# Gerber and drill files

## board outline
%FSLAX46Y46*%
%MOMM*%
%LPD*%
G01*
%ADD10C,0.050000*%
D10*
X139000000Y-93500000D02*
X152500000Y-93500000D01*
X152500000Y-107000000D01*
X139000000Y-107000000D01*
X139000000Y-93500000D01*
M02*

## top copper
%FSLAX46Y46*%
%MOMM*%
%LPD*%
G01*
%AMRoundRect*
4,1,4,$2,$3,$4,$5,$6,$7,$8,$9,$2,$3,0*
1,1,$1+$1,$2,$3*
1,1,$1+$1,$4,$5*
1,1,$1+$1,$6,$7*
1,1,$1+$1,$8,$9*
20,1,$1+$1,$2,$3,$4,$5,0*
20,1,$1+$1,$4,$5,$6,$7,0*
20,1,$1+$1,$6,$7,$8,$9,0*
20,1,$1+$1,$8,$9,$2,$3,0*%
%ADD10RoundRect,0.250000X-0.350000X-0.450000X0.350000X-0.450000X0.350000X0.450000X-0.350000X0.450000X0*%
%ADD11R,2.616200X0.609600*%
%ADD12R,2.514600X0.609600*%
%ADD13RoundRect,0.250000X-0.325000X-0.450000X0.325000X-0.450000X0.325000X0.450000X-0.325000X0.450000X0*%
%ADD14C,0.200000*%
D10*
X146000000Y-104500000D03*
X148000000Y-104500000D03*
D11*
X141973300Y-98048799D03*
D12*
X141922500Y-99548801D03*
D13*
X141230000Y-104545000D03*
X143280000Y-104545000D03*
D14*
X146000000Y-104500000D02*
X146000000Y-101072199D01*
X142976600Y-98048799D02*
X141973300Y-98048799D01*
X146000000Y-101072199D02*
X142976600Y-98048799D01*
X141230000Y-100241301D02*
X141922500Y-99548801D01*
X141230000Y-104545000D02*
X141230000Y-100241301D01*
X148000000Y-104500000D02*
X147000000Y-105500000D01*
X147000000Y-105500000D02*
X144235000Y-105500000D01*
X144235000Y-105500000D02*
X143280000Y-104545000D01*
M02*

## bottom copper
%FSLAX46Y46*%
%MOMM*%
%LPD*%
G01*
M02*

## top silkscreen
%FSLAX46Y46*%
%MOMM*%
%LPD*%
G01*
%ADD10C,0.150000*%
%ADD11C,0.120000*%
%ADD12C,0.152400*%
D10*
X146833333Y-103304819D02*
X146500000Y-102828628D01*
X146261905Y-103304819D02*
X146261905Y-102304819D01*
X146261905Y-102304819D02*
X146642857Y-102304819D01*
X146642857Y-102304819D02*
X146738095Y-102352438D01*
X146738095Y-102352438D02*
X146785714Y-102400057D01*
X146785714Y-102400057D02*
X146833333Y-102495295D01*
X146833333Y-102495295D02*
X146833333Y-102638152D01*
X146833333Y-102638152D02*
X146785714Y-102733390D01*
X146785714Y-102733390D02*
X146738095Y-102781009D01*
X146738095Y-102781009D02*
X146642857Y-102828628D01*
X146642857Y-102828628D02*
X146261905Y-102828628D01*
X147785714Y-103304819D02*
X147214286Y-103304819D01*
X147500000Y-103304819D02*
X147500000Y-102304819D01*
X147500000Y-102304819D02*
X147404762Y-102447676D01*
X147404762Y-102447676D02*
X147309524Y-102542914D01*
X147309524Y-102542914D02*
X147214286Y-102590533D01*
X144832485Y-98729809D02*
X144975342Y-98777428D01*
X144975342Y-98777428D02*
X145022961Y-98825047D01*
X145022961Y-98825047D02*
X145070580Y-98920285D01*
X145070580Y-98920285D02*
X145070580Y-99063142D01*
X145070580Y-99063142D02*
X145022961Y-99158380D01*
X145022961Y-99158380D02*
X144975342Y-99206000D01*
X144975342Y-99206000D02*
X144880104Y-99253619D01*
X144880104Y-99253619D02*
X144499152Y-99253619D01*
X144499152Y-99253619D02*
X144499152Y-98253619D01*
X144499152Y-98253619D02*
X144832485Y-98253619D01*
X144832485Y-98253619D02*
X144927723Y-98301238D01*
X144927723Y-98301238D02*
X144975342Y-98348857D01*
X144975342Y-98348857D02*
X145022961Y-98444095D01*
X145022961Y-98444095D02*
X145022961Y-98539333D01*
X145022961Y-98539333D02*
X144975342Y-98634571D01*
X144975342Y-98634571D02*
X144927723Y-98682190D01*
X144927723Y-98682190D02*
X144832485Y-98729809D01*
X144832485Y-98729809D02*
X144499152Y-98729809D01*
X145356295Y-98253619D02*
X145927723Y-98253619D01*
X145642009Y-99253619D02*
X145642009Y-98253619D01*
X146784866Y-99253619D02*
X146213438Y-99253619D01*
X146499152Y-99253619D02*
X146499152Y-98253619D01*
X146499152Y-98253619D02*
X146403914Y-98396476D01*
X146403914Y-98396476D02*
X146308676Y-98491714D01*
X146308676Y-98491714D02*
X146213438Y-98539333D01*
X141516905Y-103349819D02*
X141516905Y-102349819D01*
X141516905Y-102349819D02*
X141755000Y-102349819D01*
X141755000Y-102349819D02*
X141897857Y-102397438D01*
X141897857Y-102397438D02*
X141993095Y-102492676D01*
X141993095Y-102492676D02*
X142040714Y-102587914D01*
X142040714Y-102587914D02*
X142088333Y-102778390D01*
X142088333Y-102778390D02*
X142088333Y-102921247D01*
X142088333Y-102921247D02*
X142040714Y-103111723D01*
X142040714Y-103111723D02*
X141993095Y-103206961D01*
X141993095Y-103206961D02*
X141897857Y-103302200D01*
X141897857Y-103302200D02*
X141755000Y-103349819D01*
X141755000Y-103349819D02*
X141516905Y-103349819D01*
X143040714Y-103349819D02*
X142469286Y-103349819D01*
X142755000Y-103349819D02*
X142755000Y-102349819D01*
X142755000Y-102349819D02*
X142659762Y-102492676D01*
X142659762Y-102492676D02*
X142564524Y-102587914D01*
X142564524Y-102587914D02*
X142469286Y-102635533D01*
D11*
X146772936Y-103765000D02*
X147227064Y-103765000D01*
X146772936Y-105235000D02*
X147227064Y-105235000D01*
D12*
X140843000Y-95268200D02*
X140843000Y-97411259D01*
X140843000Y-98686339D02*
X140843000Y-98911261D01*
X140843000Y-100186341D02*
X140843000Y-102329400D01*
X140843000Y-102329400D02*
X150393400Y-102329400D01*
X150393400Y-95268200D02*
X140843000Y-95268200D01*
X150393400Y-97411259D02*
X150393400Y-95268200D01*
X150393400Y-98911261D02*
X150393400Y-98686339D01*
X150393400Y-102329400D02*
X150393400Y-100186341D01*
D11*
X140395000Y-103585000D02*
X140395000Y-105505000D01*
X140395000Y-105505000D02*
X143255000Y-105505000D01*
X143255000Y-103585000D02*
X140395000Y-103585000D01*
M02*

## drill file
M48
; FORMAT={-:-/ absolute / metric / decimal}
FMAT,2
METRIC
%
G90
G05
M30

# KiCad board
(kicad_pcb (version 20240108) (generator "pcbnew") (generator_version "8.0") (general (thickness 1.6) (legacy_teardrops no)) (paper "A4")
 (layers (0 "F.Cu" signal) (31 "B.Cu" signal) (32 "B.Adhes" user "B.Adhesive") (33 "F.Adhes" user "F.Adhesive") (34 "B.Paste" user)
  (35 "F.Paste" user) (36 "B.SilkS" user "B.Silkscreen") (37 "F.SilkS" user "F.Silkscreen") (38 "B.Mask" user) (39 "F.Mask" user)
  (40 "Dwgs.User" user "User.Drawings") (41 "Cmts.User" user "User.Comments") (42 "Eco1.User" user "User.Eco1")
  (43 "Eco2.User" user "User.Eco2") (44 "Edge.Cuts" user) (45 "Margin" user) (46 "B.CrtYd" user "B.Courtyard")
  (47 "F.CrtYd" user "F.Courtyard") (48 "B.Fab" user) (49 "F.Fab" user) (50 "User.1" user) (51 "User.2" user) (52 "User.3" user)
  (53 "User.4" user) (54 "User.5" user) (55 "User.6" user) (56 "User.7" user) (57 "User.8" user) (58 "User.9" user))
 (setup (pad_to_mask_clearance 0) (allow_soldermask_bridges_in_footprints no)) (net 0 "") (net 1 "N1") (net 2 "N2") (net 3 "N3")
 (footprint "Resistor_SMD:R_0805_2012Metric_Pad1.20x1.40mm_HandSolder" (layer "F.Cu") (at 147 104.5)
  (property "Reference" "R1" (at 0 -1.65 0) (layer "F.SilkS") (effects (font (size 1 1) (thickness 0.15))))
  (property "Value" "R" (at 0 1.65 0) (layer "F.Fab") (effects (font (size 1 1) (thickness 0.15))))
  (fp_line (start -0.227064 -0.735) (end 0.227064 -0.735) (stroke (width 0.12) (type solid)) (layer "F.SilkS"))
  (fp_line (start -0.227064 0.735) (end 0.227064 0.735) (stroke (width 0.12) (type solid)) (layer "F.SilkS"))
  (pad "1" smd roundrect (at -1 0) (size 1.2 1.4) (layers "F.Cu" "F.Paste" "F.Mask") (roundrect_rratio 0.208333) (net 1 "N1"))
  (pad "2" smd roundrect (at 1 0) (size 1.2 1.4) (layers "F.Cu" "F.Paste" "F.Mask") (roundrect_rratio 0.208333) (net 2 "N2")))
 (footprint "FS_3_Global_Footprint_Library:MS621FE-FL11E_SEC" (layer "F.Cu") (at 145.6182 98.7988)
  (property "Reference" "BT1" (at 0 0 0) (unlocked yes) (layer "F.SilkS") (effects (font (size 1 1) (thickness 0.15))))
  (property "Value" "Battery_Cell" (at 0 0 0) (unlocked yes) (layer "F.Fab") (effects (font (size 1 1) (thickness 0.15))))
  (fp_line (start -4.7752 -3.5306) (end -4.7752 -1.387541) (stroke (width 0.1524) (type solid)) (layer "F.SilkS"))
  (fp_line (start -4.7752 -0.112461) (end -4.7752 0.112461) (stroke (width 0.1524) (type solid)) (layer "F.SilkS"))
  (fp_line (start -4.7752 1.387541) (end -4.7752 3.5306) (stroke (width 0.1524) (type solid)) (layer "F.SilkS"))
  (fp_line (start -4.7752 3.5306) (end 4.7752 3.5306) (stroke (width 0.1524) (type solid)) (layer "F.SilkS"))
  (fp_line (start 4.7752 -3.5306) (end -4.7752 -3.5306) (stroke (width 0.1524) (type solid)) (layer "F.SilkS"))
  (fp_line (start 4.7752 -1.387541) (end 4.7752 -3.5306) (stroke (width 0.1524) (type solid)) (layer "F.SilkS"))
  (fp_line (start 4.7752 0.112461) (end 4.7752 -0.112461) (stroke (width 0.1524) (type solid)) (layer "F.SilkS"))
  (fp_line (start 4.7752 3.5306) (end 4.7752 1.387541) (stroke (width 0.1524) (type solid)) (layer "F.SilkS"))
  (pad "1" smd rect (at -3.6449 -0.750001) (size 2.6162 0.6096) (layers "F.Cu" "F.Paste" "F.Mask") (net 1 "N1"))
  (pad "2" smd rect (at -3.6957 0.750001) (size 2.5146 0.6096) (layers "F.Cu" "F.Paste" "F.Mask") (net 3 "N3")))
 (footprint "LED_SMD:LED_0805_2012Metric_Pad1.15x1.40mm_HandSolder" (layer "F.Cu") (at 142.255 104.545)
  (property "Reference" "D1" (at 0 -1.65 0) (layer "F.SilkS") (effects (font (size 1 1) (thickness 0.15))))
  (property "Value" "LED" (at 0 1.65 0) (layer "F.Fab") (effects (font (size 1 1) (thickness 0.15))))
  (fp_line (start -1.86 -0.96) (end -1.86 0.96) (stroke (width 0.12) (type solid)) (layer "F.SilkS"))
  (fp_line (start -1.86 0.96) (end 1 0.96) (stroke (width 0.12) (type solid)) (layer "F.SilkS"))
  (fp_line (start 1 -0.96) (end -1.86 -0.96) (stroke (width 0.12) (type solid)) (layer "F.SilkS"))
  (pad "1" smd roundrect (at -1.025 0) (size 1.15 1.4) (layers "F.Cu" "F.Paste" "F.Mask") (roundrect_rratio 0.217391) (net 3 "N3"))
  (pad "2" smd roundrect (at 1.025 0) (size 1.15 1.4) (layers "F.Cu" "F.Paste" "F.Mask") (roundrect_rratio 0.217391) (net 2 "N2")))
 (gr_rect (start 139 93.5) (end 152.5 107) (stroke (width 0.05) (type default)) (fill none) (layer "Edge.Cuts"))
 (segment (start 146 104.5) (end 146 101.072199) (width 0.2) (layer "F.Cu") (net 1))
 (segment (start 142.9766 98.048799) (end 141.9733 98.048799) (width 0.2) (layer "F.Cu") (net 1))
 (segment (start 146 101.072199) (end 142.9766 98.048799) (width 0.2) (layer "F.Cu") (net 1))
 (segment (start 141.23 100.241301) (end 141.9225 99.548801) (width 0.2) (layer "F.Cu") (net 3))
 (segment (start 141.23 104.545) (end 141.23 100.241301) (width 0.2) (layer "F.Cu") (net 3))
 (segment (start 148 104.5) (end 147 105.5) (width 0.2) (layer "F.Cu") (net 2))
 (segment (start 147 105.5) (end 144.235 105.5) (width 0.2) (layer "F.Cu") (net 2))
 (segment (start 144.235 105.5) (end 143.28 104.545) (width 0.2) (layer "F.Cu") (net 2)))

